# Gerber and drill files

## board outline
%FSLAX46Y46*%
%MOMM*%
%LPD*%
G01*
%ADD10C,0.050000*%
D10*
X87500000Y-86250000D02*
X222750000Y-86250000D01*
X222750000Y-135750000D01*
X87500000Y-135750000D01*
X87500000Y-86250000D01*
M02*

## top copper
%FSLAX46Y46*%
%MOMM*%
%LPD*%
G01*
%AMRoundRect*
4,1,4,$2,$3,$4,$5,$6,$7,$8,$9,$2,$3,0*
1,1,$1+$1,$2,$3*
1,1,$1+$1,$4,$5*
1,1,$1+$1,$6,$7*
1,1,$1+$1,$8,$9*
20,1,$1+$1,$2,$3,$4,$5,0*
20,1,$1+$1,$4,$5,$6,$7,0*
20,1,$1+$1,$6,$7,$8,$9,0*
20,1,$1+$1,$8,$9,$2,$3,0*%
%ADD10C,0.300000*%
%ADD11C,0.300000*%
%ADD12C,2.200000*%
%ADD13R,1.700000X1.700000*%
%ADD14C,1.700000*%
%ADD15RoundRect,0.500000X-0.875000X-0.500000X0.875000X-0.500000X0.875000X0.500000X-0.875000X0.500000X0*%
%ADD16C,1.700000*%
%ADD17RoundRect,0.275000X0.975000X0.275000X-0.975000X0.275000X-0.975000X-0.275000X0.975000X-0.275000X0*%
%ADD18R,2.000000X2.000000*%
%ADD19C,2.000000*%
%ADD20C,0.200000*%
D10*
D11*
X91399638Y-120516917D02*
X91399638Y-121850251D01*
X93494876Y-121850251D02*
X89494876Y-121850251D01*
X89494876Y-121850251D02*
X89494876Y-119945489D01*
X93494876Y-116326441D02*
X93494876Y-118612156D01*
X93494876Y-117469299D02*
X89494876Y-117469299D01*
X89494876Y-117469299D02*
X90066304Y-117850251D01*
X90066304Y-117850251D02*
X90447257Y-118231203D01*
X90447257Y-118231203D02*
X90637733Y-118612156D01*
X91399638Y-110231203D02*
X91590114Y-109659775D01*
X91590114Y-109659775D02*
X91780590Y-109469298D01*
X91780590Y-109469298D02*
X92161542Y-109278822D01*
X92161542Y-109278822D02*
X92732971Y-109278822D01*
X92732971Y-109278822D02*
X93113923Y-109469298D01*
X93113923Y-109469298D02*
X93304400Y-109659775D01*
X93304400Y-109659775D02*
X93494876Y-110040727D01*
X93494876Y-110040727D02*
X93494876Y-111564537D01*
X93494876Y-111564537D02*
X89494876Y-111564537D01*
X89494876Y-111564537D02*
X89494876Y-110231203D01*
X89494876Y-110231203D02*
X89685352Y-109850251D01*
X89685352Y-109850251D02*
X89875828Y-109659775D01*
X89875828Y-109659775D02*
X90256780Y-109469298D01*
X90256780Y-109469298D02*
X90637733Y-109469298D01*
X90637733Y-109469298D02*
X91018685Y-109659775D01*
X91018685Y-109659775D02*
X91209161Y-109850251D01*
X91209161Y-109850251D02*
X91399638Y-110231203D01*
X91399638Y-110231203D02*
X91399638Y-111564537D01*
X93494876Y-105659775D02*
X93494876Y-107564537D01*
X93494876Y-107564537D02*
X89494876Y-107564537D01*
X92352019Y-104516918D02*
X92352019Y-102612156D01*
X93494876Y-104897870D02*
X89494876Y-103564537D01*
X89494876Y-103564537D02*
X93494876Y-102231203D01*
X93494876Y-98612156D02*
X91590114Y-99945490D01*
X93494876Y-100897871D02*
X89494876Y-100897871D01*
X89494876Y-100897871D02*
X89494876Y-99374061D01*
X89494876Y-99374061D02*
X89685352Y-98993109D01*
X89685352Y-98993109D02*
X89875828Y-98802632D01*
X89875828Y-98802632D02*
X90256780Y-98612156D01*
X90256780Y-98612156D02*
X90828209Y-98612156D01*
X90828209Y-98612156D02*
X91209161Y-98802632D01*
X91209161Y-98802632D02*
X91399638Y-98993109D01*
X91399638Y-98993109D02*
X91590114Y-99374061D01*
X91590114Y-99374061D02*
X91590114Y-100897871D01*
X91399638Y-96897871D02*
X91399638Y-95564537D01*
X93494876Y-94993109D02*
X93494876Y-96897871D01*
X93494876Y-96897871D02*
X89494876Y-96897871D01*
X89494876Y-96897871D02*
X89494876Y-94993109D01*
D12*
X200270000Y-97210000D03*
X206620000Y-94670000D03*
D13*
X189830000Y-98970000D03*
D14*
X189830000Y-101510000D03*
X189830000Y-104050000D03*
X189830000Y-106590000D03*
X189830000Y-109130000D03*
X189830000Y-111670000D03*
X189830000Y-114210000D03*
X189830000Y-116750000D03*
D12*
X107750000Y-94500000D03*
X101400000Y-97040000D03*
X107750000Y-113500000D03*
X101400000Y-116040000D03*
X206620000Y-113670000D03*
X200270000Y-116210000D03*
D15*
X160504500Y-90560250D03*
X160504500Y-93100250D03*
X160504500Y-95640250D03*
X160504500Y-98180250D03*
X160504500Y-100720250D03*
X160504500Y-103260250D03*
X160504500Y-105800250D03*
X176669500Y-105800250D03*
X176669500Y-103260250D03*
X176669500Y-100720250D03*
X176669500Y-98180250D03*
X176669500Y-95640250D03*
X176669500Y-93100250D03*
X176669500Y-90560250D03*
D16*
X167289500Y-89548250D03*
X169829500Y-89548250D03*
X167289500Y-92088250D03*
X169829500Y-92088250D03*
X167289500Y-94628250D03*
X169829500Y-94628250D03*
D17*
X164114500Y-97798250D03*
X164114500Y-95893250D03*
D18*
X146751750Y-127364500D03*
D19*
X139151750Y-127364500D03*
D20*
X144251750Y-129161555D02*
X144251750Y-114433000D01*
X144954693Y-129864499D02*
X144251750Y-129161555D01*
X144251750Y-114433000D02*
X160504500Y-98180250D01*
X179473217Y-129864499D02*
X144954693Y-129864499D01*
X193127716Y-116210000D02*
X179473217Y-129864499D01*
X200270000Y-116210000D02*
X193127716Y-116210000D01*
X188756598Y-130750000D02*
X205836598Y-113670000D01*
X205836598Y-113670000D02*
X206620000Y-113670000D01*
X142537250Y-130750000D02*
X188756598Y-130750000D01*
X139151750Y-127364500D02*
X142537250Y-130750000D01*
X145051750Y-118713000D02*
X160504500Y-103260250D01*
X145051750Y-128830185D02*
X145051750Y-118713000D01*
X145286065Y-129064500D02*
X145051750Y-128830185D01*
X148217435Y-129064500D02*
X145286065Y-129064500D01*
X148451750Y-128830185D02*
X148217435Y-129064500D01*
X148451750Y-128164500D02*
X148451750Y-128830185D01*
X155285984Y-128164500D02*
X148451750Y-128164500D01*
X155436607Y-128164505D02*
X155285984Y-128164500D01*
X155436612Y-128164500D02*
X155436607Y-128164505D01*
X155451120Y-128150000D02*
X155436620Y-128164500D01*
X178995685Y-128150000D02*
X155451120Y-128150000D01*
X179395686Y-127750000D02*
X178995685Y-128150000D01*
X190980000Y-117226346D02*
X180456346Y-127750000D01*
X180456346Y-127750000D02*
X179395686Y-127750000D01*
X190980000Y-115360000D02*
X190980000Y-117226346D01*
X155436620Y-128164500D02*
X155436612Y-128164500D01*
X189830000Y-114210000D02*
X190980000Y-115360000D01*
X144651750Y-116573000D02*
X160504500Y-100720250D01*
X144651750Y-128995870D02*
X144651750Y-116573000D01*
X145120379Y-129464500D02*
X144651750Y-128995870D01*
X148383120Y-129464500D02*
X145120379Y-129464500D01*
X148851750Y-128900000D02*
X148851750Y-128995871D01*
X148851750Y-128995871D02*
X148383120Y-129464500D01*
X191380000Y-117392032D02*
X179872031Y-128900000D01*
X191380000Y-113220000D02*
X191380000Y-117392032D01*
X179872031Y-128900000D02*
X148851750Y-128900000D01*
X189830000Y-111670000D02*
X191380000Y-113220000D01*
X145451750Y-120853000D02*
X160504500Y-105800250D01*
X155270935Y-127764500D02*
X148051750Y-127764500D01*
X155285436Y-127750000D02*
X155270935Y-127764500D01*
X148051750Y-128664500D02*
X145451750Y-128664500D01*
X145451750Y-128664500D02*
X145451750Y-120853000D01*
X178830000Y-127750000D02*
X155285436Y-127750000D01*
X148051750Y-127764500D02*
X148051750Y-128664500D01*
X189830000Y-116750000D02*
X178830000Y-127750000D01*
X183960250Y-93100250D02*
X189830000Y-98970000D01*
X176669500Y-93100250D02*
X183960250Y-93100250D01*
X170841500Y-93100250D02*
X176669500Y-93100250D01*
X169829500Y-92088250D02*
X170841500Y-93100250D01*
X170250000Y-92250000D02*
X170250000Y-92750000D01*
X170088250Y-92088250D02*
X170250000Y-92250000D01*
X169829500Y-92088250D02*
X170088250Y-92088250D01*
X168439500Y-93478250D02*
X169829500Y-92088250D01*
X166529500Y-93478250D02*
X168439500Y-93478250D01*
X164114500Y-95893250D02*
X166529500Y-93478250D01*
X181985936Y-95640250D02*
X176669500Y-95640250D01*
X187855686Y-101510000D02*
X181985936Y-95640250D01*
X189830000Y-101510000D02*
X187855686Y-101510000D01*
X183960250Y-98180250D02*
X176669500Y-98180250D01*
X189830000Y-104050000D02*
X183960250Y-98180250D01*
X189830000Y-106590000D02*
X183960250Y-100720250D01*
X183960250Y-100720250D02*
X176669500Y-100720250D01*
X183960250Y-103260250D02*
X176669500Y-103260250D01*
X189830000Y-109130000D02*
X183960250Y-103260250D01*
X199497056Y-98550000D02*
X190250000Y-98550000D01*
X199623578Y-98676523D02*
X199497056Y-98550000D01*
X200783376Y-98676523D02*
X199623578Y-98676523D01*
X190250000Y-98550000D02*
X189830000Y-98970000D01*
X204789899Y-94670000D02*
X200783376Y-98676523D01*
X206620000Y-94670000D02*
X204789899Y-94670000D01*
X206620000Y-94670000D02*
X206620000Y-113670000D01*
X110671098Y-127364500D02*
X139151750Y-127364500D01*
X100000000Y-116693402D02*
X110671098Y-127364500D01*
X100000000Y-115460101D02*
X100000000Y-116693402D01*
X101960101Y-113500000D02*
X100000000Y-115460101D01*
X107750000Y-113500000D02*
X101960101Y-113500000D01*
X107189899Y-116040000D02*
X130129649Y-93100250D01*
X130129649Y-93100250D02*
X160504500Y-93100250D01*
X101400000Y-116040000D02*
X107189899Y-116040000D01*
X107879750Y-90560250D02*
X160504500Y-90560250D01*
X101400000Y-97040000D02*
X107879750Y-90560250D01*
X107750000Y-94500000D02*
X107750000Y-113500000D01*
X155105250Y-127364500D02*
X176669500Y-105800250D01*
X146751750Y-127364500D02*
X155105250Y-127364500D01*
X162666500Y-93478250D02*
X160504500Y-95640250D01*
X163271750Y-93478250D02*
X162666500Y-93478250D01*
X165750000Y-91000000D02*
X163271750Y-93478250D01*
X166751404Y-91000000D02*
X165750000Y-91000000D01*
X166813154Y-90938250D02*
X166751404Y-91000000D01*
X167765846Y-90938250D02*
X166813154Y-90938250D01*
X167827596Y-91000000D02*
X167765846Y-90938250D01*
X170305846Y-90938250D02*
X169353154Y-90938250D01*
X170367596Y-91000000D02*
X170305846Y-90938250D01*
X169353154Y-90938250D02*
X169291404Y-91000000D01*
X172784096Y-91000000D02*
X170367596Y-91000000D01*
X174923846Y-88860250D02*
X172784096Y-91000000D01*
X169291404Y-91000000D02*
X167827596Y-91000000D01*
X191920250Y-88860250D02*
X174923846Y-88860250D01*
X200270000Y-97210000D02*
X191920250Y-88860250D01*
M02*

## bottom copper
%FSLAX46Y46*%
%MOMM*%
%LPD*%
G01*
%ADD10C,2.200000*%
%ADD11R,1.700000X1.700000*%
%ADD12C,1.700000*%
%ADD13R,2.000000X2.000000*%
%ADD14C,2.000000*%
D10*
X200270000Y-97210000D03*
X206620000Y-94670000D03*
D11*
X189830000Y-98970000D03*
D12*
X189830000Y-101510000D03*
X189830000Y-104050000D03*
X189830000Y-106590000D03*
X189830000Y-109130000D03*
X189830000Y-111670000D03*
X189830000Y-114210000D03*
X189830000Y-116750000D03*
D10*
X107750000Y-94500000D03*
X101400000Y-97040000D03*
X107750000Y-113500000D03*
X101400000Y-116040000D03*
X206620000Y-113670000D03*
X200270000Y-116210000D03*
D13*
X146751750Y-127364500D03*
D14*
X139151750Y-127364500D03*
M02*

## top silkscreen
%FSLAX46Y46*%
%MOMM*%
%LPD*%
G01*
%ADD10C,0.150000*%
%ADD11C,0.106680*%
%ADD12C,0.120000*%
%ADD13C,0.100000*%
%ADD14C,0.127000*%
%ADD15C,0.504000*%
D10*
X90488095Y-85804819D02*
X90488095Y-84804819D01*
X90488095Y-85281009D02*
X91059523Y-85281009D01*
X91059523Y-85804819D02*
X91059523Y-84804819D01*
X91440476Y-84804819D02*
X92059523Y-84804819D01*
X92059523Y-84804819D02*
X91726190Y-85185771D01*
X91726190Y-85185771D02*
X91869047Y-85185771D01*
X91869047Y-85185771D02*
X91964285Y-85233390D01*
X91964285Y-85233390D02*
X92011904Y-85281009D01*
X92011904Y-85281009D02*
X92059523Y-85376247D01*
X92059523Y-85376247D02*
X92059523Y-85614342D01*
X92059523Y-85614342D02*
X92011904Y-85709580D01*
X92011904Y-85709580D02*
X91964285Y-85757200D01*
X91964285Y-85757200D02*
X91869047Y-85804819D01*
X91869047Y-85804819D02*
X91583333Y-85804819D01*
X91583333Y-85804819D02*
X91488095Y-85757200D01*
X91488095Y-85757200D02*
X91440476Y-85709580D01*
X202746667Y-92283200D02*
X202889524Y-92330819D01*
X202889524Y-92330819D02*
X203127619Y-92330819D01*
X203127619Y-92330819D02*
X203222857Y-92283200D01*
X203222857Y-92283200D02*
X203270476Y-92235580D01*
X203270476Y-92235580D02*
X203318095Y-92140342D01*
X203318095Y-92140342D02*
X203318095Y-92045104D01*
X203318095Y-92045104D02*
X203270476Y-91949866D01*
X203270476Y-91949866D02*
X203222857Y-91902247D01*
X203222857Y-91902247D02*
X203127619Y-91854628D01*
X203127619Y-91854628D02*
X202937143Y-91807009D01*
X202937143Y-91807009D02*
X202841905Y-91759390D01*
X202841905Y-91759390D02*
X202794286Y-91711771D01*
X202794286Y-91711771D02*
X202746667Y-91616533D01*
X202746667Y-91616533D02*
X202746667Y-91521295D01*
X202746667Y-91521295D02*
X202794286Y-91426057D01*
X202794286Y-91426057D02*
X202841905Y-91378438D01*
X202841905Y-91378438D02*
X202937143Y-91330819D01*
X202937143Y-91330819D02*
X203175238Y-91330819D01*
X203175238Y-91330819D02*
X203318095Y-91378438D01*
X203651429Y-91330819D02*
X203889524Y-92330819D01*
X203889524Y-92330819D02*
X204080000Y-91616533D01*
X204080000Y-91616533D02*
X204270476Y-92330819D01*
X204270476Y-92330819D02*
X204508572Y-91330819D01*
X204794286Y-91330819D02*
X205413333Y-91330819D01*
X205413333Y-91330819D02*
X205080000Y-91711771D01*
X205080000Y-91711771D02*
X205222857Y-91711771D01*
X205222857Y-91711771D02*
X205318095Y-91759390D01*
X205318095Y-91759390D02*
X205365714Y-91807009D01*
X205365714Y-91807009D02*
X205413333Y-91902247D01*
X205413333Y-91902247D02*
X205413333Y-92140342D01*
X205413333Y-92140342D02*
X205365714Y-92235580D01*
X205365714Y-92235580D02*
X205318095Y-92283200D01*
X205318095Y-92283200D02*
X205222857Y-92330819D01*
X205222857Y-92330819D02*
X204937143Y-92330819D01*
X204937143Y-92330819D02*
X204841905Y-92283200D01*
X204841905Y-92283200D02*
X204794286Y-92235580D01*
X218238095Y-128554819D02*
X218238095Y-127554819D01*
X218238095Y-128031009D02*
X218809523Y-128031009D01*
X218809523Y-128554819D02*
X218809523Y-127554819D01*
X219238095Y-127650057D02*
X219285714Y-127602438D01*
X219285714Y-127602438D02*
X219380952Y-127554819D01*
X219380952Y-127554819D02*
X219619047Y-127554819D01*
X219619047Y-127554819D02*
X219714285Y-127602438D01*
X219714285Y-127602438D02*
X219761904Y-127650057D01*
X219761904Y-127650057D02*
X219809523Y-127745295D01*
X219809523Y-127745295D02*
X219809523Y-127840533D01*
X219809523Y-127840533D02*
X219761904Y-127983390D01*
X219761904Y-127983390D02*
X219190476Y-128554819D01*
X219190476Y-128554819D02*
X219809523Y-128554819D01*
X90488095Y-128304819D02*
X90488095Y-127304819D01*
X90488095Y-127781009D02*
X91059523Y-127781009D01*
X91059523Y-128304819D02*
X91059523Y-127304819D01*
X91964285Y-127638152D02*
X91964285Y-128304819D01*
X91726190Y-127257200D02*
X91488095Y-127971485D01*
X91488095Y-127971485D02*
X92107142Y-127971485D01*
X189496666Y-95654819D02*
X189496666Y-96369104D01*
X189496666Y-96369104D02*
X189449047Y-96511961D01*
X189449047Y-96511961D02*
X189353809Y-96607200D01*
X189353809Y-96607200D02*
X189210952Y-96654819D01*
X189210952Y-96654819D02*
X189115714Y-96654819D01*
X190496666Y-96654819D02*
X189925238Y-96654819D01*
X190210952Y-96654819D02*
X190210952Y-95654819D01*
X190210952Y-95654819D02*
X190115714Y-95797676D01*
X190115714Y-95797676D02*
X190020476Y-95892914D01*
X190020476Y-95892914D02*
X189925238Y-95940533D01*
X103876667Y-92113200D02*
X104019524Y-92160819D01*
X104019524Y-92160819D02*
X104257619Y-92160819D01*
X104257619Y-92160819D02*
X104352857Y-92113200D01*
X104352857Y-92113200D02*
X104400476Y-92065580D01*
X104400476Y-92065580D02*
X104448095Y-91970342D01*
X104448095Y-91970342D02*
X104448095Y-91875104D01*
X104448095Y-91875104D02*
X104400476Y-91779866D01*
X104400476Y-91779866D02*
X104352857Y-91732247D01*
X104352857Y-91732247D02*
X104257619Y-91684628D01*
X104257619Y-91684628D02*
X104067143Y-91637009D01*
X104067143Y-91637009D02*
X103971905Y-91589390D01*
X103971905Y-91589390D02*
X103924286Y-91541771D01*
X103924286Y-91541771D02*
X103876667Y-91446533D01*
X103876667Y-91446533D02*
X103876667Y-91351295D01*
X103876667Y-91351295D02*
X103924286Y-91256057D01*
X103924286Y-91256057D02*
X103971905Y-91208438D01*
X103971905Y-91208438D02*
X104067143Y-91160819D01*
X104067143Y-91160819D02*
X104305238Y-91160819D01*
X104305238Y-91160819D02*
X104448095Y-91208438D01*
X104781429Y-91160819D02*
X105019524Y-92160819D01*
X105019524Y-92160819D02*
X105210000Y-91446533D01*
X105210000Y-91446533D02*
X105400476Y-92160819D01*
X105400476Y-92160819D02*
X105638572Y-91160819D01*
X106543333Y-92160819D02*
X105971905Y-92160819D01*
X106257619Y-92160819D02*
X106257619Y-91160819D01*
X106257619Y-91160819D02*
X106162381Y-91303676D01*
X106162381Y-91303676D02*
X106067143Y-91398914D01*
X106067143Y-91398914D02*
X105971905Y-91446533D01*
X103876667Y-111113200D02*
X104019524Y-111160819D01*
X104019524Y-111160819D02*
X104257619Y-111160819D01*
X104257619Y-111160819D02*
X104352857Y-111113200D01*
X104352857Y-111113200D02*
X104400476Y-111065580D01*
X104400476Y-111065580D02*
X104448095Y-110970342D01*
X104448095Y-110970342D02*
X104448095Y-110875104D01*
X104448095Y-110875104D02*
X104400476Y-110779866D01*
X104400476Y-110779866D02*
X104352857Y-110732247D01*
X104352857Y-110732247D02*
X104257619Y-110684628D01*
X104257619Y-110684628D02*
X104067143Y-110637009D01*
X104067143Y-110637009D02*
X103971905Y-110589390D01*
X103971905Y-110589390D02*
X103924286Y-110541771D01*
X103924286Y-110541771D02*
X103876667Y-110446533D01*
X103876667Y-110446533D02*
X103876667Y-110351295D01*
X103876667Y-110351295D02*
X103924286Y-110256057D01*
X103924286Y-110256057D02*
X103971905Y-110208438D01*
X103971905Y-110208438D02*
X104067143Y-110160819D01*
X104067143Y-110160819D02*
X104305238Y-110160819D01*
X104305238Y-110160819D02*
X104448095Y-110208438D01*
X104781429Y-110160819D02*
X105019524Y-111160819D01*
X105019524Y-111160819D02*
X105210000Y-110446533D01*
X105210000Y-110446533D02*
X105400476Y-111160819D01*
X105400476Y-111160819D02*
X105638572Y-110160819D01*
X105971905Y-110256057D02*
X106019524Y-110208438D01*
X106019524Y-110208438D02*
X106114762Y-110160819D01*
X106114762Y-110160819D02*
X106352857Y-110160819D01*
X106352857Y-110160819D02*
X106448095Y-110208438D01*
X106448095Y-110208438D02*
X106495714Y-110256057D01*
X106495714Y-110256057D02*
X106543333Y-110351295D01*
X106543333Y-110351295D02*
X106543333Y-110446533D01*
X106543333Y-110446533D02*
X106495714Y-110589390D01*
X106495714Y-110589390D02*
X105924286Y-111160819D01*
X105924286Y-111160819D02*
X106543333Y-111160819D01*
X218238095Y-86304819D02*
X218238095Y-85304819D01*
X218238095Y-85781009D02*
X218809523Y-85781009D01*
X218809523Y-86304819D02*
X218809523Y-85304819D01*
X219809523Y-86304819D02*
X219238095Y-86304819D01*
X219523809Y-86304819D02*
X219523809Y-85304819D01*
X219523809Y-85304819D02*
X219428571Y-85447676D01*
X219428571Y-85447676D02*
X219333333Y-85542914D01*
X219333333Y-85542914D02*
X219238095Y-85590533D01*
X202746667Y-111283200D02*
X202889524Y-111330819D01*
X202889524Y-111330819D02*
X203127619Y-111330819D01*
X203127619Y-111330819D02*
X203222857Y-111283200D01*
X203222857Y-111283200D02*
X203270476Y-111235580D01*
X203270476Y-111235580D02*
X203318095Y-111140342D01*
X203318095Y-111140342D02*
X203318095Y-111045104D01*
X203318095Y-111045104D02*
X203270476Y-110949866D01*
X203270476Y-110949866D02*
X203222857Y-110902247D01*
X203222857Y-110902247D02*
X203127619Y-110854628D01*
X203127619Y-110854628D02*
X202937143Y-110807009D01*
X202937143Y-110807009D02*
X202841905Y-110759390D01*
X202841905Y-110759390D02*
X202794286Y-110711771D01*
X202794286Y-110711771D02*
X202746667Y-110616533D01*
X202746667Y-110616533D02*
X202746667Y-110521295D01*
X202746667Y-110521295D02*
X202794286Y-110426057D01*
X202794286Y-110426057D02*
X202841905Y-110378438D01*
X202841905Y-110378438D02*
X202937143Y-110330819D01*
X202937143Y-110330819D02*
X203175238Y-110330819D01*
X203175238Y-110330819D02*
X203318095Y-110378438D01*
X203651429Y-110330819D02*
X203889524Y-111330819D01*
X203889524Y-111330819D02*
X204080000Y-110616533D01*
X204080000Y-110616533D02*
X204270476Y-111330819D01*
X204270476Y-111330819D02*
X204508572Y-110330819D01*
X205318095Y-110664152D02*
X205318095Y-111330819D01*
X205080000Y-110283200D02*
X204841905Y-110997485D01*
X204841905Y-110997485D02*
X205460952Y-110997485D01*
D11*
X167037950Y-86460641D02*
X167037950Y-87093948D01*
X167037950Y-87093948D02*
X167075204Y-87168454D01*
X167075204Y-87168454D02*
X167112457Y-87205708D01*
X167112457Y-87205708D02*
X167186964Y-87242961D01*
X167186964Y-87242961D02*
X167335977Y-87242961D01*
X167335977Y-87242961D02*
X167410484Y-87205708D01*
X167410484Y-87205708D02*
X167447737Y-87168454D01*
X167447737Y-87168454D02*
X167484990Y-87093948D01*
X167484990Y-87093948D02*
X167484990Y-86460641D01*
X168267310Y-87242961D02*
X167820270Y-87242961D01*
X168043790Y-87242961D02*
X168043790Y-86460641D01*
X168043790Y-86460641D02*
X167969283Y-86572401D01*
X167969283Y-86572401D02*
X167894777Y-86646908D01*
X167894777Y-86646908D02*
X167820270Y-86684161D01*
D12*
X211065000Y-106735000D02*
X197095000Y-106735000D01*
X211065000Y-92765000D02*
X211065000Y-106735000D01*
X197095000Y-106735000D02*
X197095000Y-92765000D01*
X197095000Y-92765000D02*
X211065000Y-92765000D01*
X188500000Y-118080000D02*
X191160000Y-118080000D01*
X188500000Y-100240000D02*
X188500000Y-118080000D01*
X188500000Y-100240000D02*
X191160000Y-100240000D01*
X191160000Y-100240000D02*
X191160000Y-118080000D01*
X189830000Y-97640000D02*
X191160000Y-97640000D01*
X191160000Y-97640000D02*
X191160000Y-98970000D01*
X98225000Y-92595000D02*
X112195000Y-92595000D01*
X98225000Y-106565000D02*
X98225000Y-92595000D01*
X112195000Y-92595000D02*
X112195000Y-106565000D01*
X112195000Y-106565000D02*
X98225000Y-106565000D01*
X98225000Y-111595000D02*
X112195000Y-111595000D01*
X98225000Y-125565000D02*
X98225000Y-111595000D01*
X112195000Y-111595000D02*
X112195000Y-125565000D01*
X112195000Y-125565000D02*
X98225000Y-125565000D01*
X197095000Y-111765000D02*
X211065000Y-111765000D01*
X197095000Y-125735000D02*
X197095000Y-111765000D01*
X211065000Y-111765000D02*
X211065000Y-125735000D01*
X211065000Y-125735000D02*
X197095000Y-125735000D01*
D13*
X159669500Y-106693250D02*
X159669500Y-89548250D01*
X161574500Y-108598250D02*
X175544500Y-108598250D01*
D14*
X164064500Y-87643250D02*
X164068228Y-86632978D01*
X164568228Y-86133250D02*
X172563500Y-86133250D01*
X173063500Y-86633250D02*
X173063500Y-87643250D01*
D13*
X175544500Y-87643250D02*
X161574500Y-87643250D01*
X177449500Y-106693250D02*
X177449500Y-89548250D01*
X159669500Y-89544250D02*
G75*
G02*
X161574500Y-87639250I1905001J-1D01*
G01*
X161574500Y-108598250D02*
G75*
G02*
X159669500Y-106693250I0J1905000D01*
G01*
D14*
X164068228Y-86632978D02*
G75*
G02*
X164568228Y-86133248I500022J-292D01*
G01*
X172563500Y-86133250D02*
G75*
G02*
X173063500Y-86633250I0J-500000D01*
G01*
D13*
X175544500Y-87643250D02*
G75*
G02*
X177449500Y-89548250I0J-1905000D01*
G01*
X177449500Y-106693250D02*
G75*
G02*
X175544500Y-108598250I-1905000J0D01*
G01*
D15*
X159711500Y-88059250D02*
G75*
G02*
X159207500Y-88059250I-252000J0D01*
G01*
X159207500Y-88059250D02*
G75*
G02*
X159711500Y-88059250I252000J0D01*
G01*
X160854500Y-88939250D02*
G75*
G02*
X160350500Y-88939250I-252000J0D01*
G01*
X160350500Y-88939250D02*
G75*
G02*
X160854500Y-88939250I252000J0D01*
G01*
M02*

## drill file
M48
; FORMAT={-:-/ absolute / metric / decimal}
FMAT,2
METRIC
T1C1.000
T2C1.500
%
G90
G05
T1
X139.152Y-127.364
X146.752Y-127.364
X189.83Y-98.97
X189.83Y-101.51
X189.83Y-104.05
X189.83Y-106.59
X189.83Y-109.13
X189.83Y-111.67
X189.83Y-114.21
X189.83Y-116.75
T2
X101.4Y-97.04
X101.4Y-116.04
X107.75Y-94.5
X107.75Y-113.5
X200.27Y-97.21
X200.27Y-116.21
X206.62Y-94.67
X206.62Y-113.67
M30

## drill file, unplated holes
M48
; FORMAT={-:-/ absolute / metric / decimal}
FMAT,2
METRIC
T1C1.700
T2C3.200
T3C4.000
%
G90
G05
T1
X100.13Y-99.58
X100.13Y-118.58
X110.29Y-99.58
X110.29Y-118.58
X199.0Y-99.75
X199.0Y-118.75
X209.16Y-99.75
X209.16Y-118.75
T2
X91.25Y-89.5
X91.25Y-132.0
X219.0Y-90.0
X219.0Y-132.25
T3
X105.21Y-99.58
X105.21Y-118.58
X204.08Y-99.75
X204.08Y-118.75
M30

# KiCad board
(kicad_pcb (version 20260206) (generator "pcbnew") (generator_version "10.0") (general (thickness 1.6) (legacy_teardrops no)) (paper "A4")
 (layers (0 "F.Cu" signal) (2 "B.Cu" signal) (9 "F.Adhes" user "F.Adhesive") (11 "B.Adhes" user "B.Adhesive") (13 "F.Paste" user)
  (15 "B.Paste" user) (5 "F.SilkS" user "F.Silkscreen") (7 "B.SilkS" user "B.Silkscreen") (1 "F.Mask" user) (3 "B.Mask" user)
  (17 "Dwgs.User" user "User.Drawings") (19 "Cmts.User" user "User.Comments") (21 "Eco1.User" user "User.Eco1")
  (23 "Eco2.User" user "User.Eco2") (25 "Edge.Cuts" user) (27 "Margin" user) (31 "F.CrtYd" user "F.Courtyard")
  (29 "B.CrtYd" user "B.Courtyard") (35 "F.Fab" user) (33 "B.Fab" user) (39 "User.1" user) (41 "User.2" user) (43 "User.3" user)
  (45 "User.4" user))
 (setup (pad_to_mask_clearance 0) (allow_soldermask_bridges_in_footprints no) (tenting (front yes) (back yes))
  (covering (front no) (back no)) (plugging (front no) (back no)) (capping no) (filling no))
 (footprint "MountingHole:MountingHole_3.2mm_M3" (layer "F.Cu") (at 219 132.25)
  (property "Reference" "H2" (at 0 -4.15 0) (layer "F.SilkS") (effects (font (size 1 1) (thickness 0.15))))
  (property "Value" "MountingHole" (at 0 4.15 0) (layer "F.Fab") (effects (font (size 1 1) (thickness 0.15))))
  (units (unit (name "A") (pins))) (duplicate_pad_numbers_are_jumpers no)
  (pad "" np_thru_hole circle (at 0 0) (size 3.2 3.2) (drill 3.2) (layers "*.Cu" "*.Mask")))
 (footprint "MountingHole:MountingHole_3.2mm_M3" (layer "F.Cu") (at 91.25 132)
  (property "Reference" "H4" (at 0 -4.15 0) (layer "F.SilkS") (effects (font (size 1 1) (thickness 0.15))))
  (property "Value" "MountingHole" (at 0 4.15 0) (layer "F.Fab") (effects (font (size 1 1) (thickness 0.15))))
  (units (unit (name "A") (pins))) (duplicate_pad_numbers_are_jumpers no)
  (pad "" np_thru_hole circle (at 0 0) (size 3.2 3.2) (drill 3.2) (layers "*.Cu" "*.Mask")))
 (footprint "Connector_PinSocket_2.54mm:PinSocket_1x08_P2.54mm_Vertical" (layer "F.Cu") (at 189.83 98.97)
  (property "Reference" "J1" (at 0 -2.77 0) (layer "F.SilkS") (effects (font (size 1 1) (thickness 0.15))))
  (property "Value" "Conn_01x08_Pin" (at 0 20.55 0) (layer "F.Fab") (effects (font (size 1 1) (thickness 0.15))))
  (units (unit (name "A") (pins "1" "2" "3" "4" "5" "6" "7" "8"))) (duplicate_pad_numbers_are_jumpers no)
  (fp_line (start -1.33 1.27) (end -1.33 19.11) (stroke (width 0.12) (type solid)) (layer "F.SilkS"))
  (fp_line (start -1.33 1.27) (end 1.33 1.27) (stroke (width 0.12) (type solid)) (layer "F.SilkS"))
  (fp_line (start -1.33 19.11) (end 1.33 19.11) (stroke (width 0.12) (type solid)) (layer "F.SilkS"))
  (fp_line (start 0 -1.33) (end 1.33 -1.33) (stroke (width 0.12) (type solid)) (layer "F.SilkS"))
  (fp_line (start 1.33 -1.33) (end 1.33 0) (stroke (width 0.12) (type solid)) (layer "F.SilkS"))
  (fp_line (start 1.33 1.27) (end 1.33 19.11) (stroke (width 0.12) (type solid)) (layer "F.SilkS"))
  (pad "1" thru_hole rect (at 0 0) (size 1.7 1.7) (drill 1) (layers "*.Cu" "*.Mask") (remove_unused_layers no) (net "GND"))
  (pad "2" thru_hole circle (at 0 2.54) (size 1.7 1.7) (drill 1) (layers "*.Cu" "*.Mask") (remove_unused_layers no) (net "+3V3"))
  (pad "3" thru_hole circle (at 0 5.08) (size 1.7 1.7) (drill 1) (layers "*.Cu" "*.Mask") (remove_unused_layers no) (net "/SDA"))
  (pad "4" thru_hole circle (at 0 7.62) (size 1.7 1.7) (drill 1) (layers "*.Cu" "*.Mask") (remove_unused_layers no) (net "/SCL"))
  (pad "5" thru_hole circle (at 0 10.16) (size 1.7 1.7) (drill 1) (layers "*.Cu" "*.Mask") (remove_unused_layers no) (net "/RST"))
  (pad "6" thru_hole circle (at 0 12.7) (size 1.7 1.7) (drill 1) (layers "*.Cu" "*.Mask") (remove_unused_layers no) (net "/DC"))
  (pad "7" thru_hole circle (at 0 15.24) (size 1.7 1.7) (drill 1) (layers "*.Cu" "*.Mask") (remove_unused_layers no) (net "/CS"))
  (pad "8" thru_hole circle (at 0 17.78) (size 1.7 1.7) (drill 1) (layers "*.Cu" "*.Mask") (remove_unused_layers no) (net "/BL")))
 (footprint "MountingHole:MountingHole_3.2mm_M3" (layer "F.Cu") (at 91.25 89.5)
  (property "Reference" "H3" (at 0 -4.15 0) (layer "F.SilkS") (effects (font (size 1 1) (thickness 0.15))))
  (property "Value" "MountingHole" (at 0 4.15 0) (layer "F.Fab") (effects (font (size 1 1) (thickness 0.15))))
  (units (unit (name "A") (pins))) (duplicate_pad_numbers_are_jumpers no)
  (pad "" np_thru_hole circle (at 0 0) (size 3.2 3.2) (drill 3.2) (layers "*.Cu" "*.Mask")))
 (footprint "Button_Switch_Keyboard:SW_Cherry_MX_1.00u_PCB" (layer "F.Cu") (at 206.62 94.67)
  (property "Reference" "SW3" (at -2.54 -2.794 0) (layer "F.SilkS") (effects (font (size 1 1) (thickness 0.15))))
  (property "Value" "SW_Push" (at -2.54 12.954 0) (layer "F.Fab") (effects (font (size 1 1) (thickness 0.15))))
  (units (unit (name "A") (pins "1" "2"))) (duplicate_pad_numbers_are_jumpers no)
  (fp_line (start -9.525 -1.905) (end 4.445 -1.905) (stroke (width 0.12) (type solid)) (layer "F.SilkS"))
  (fp_line (start -9.525 12.065) (end -9.525 -1.905) (stroke (width 0.12) (type solid)) (layer "F.SilkS"))
  (fp_line (start 4.445 -1.905) (end 4.445 12.065) (stroke (width 0.12) (type solid)) (layer "F.SilkS"))
  (fp_line (start 4.445 12.065) (end -9.525 12.065) (stroke (width 0.12) (type solid)) (layer "F.SilkS"))
  (pad "" np_thru_hole circle (at -7.62 5.08) (size 1.7 1.7) (drill 1.7) (layers "*.Cu" "*.Mask"))
  (pad "" np_thru_hole circle (at -2.54 5.08) (size 4 4) (drill 4) (layers "*.Cu" "*.Mask"))
  (pad "" np_thru_hole circle (at 2.54 5.08) (size 1.7 1.7) (drill 1.7) (layers "*.Cu" "*.Mask"))
  (pad "1" thru_hole circle (at 0 0) (size 2.2 2.2) (drill 1.5) (layers "*.Cu" "*.Mask") (remove_unused_layers no) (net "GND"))
  (pad "2" thru_hole circle (at -6.35 2.54) (size 2.2 2.2) (drill 1.5) (layers "*.Cu" "*.Mask") (remove_unused_layers no)
   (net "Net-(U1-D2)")))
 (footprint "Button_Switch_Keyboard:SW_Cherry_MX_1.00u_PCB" (layer "F.Cu") (at 107.75 94.5)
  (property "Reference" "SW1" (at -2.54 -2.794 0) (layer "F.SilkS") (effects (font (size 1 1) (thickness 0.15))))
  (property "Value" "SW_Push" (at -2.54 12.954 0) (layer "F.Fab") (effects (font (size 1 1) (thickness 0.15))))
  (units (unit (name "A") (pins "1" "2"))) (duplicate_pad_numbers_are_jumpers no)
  (fp_line (start -9.525 -1.905) (end 4.445 -1.905) (stroke (width 0.12) (type solid)) (layer "F.SilkS"))
  (fp_line (start -9.525 12.065) (end -9.525 -1.905) (stroke (width 0.12) (type solid)) (layer "F.SilkS"))
  (fp_line (start 4.445 -1.905) (end 4.445 12.065) (stroke (width 0.12) (type solid)) (layer "F.SilkS"))
  (fp_line (start 4.445 12.065) (end -9.525 12.065) (stroke (width 0.12) (type solid)) (layer "F.SilkS"))
  (pad "" np_thru_hole circle (at -7.62 5.08) (size 1.7 1.7) (drill 1.7) (layers "*.Cu" "*.Mask"))
  (pad "" np_thru_hole circle (at -2.54 5.08) (size 4 4) (drill 4) (layers "*.Cu" "*.Mask"))
  (pad "" np_thru_hole circle (at 2.54 5.08) (size 1.7 1.7) (drill 1.7) (layers "*.Cu" "*.Mask"))
  (pad "1" thru_hole circle (at 0 0) (size 2.2 2.2) (drill 1.5) (layers "*.Cu" "*.Mask") (remove_unused_layers no) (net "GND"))
  (pad "2" thru_hole circle (at -6.35 2.54) (size 2.2 2.2) (drill 1.5) (layers "*.Cu" "*.Mask") (remove_unused_layers no)
   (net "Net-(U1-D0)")))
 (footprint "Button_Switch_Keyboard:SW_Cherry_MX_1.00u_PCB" (layer "F.Cu") (at 107.75 113.5)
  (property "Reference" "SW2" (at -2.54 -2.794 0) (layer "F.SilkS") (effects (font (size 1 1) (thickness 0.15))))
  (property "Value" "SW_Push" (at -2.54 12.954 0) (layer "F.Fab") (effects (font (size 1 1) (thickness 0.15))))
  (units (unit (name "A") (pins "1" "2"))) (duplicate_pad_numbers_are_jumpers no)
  (fp_line (start -9.525 -1.905) (end 4.445 -1.905) (stroke (width 0.12) (type solid)) (layer "F.SilkS"))
  (fp_line (start -9.525 12.065) (end -9.525 -1.905) (stroke (width 0.12) (type solid)) (layer "F.SilkS"))
  (fp_line (start 4.445 -1.905) (end 4.445 12.065) (stroke (width 0.12) (type solid)) (layer "F.SilkS"))
  (fp_line (start 4.445 12.065) (end -9.525 12.065) (stroke (width 0.12) (type solid)) (layer "F.SilkS"))
  (pad "" np_thru_hole circle (at -7.62 5.08) (size 1.7 1.7) (drill 1.7) (layers "*.Cu" "*.Mask"))
  (pad "" np_thru_hole circle (at -2.54 5.08) (size 4 4) (drill 4) (layers "*.Cu" "*.Mask"))
  (pad "" np_thru_hole circle (at 2.54 5.08) (size 1.7 1.7) (drill 1.7) (layers "*.Cu" "*.Mask"))
  (pad "1" thru_hole circle (at 0 0) (size 2.2 2.2) (drill 1.5) (layers "*.Cu" "*.Mask") (remove_unused_layers no) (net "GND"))
  (pad "2" thru_hole circle (at -6.35 2.54) (size 2.2 2.2) (drill 1.5) (layers "*.Cu" "*.Mask") (remove_unused_layers no)
   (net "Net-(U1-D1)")))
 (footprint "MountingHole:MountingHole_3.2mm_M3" (layer "F.Cu") (at 219 90)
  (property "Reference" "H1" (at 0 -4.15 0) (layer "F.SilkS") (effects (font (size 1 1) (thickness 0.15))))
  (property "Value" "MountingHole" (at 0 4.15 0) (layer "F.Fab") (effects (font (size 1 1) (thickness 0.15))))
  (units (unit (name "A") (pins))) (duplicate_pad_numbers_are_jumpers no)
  (pad "" np_thru_hole circle (at 0 0) (size 3.2 3.2) (drill 3.2) (layers "*.Cu" "*.Mask")))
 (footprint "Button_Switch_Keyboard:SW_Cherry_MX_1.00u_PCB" (layer "F.Cu") (at 206.62 113.67)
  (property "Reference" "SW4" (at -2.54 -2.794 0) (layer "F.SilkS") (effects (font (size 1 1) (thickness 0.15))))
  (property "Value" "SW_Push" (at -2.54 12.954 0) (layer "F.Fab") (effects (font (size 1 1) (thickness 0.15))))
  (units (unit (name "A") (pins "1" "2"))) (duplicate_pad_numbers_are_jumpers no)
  (fp_line (start -9.525 -1.905) (end 4.445 -1.905) (stroke (width 0.12) (type solid)) (layer "F.SilkS"))
  (fp_line (start -9.525 12.065) (end -9.525 -1.905) (stroke (width 0.12) (type solid)) (layer "F.SilkS"))
  (fp_line (start 4.445 -1.905) (end 4.445 12.065) (stroke (width 0.12) (type solid)) (layer "F.SilkS"))
  (fp_line (start 4.445 12.065) (end -9.525 12.065) (stroke (width 0.12) (type solid)) (layer "F.SilkS"))
  (pad "" np_thru_hole circle (at -7.62 5.08) (size 1.7 1.7) (drill 1.7) (layers "*.Cu" "*.Mask"))
  (pad "" np_thru_hole circle (at -2.54 5.08) (size 4 4) (drill 4) (layers "*.Cu" "*.Mask"))
  (pad "" np_thru_hole circle (at 2.54 5.08) (size 1.7 1.7) (drill 1.7) (layers "*.Cu" "*.Mask"))
  (pad "1" thru_hole circle (at 0 0) (size 2.2 2.2) (drill 1.5) (layers "*.Cu" "*.Mask") (remove_unused_layers no) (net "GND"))
  (pad "2" thru_hole circle (at -6.35 2.54) (size 2.2 2.2) (drill 1.5) (layers "*.Cu" "*.Mask") (remove_unused_layers no)
   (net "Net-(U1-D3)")))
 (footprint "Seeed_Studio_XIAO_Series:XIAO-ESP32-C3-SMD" (layer "F.Cu") (at 159.6695 108.68025)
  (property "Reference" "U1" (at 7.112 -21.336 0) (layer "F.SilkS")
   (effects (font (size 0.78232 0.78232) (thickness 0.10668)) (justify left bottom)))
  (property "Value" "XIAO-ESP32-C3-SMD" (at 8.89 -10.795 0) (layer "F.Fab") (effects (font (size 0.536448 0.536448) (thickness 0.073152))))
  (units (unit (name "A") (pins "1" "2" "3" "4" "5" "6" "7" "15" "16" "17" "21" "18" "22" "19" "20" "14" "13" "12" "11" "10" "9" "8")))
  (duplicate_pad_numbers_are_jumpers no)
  (fp_line (start 0 -1.987) (end 0 -19.132) (stroke (width 0.1) (type solid)) (layer "F.SilkS"))
  (fp_line (start 1.905 -0.082) (end 15.875 -0.082) (stroke (width 0.1) (type solid)) (layer "F.SilkS"))
  (fp_line (start 4.395 -21.037) (end 4.398728 -22.047272) (stroke (width 0.127) (type solid)) (layer "F.SilkS"))
  (fp_line (start 4.898728 -22.547) (end 12.894 -22.547) (stroke (width 0.127) (type solid)) (layer "F.SilkS"))
  (fp_line (start 13.394 -22.047) (end 13.394 -21.037) (stroke (width 0.127) (type solid)) (layer "F.SilkS"))
  (fp_line (start 15.875 -21.037) (end 1.905 -21.037) (stroke (width 0.1) (type solid)) (layer "F.SilkS"))
  (fp_line (start 17.78 -1.987) (end 17.78 -19.132) (stroke (width 0.1) (type solid)) (layer "F.SilkS"))
  (fp_arc (start 0 -19.136) (mid 0.557962 -20.483038) (end 1.905 -21.041) (stroke (width 0.1) (type solid)) (layer "F.SilkS"))
  (fp_arc (start 1.905 -0.082) (mid 0.557962 -0.639962) (end 0 -1.987) (stroke (width 0.1) (type solid)) (layer "F.SilkS"))
  (fp_arc (start 4.398728 -22.047272) (mid 4.545272 -22.40064) (end 4.898728 -22.547) (stroke (width 0.127) (type default))
   (layer "F.SilkS"))
  (fp_arc (start 12.894 -22.547) (mid 13.247553 -22.400553) (end 13.394 -22.047) (stroke (width 0.127) (type default)) (layer "F.SilkS"))
  (fp_arc (start 15.875 -21.037) (mid 17.222038 -20.479038) (end 17.78 -19.132) (stroke (width 0.1) (type solid)) (layer "F.SilkS"))
  (fp_arc (start 17.78 -1.987) (mid 17.222038 -0.639962) (end 15.875 -0.082) (stroke (width 0.1) (type solid)) (layer "F.SilkS"))
  (fp_circle (center -0.21 -20.621) (end -0.21 -20.875) (stroke (width 0.5) (type solid)) (fill yes) (layer "F.SilkS"))
  (fp_circle (center 0.933 -19.741) (end 0.933 -19.995) (stroke (width 0.5) (type solid)) (fill yes) (layer "F.SilkS"))
  (pad "1" smd roundrect (at 0.835 -18.12) (size 2.75 2) (layers "F.Cu" "F.Mask" "F.Paste") (roundrect_rratio 0.25) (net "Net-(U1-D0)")
   (solder_mask_margin 0.0508) (thermal_bridge_angle 45))
  (pad "2" smd roundrect (at 0.835 -15.58) (size 2.75 2) (layers "F.Cu" "F.Mask" "F.Paste") (roundrect_rratio 0.25) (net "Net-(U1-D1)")
   (solder_mask_margin 0.0508) (thermal_bridge_angle 45))
  (pad "3" smd roundrect (at 0.835 -13.04) (size 2.75 2) (layers "F.Cu" "F.Mask" "F.Paste") (roundrect_rratio 0.25) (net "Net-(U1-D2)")
   (solder_mask_margin 0.0508) (thermal_bridge_angle 45))
  (pad "4" smd roundrect (at 0.835 -10.5) (size 2.75 2) (layers "F.Cu" "F.Mask" "F.Paste") (roundrect_rratio 0.25) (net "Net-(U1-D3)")
   (solder_mask_margin 0.0508) (thermal_bridge_angle 45))
  (pad "5" smd roundrect (at 0.835 -7.96) (size 2.75 2) (layers "F.Cu" "F.Mask" "F.Paste") (roundrect_rratio 0.25) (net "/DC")
   (solder_mask_margin 0.0508) (thermal_bridge_angle 45))
  (pad "6" smd roundrect (at 0.835 -5.42) (size 2.75 2) (layers "F.Cu" "F.Mask" "F.Paste") (roundrect_rratio 0.25) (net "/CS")
   (solder_mask_margin 0.0508) (thermal_bridge_angle 45))
  (pad "7" smd roundrect (at 0.835 -2.88) (size 2.75 2) (layers "F.Cu" "F.Mask" "F.Paste") (roundrect_rratio 0.25) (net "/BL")
   (solder_mask_margin 0.0508) (thermal_bridge_angle 45))
  (pad "8" smd roundrect (at 17 -2.88) (size 2.75 2) (layers "F.Cu" "F.Mask" "F.Paste") (roundrect_rratio 0.25) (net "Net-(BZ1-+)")
   (solder_mask_margin 0.0508) (thermal_bridge_angle 45))
  (pad "9" smd roundrect (at 17 -5.42) (size 2.75 2) (layers "F.Cu" "F.Mask" "F.Paste") (roundrect_rratio 0.25) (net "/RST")
   (solder_mask_margin 0.0508) (thermal_bridge_angle 45))
  (pad "10" smd roundrect (at 17 -7.96) (size 2.75 2) (layers "F.Cu" "F.Mask" "F.Paste") (roundrect_rratio 0.25) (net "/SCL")
   (solder_mask_margin 0.0508) (thermal_bridge_angle 45))
  (pad "11" smd roundrect (at 17 -10.5) (size 2.75 2) (layers "F.Cu" "F.Mask" "F.Paste") (roundrect_rratio 0.25) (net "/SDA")
   (solder_mask_margin 0.0508) (thermal_bridge_angle 45))
  (pad "12" smd roundrect (at 17 -13.04) (size 2.75 2) (layers "F.Cu" "F.Mask" "F.Paste") (roundrect_rratio 0.25) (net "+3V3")
   (solder_mask_margin 0.0508) (thermal_bridge_angle 45))
  (pad "13" smd roundrect (at 17 -15.58) (size 2.75 2) (layers "F.Cu" "F.Mask" "F.Paste") (roundrect_rratio 0.25) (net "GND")
   (solder_mask_margin 0.0508) (thermal_bridge_angle 45))
  (pad "14" smd roundrect (at 17 -18.12) (size 2.75 2) (layers "F.Cu" "F.Mask" "F.Paste") (roundrect_rratio 0.25)
   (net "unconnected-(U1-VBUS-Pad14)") (solder_mask_margin 0.0508) (thermal_bridge_angle 45))
  (pad "15" smd circle (at 7.62 -19.132) (size 1.7 1.7) (layers "F.Cu" "F.Mask" "F.Paste") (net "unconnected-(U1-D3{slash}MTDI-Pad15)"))
  (pad "16" smd circle (at 10.16 -19.132) (size 1.7 1.7) (layers "F.Cu" "F.Mask" "F.Paste") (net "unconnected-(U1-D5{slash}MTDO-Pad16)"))
  (pad "17" smd circle (at 7.62 -16.592) (size 1.7 1.7) (layers "F.Cu" "F.Mask" "F.Paste") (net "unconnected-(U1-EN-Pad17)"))
  (pad "18" smd circle (at 10.16 -16.592) (size 1.7 1.7) (layers "F.Cu" "F.Mask" "F.Paste") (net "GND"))
  (pad "19" smd circle (at 7.62 -14.052) (size 1.7 1.7) (layers "F.Cu" "F.Mask" "F.Paste") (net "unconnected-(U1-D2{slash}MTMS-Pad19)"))
  (pad "20" smd circle (at 10.16 -14.052) (size 1.7 1.7) (layers "F.Cu" "F.Mask" "F.Paste") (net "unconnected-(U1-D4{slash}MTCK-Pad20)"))
  (pad "21" smd roundrect (at 4.445 -10.882 180) (size 2.5 1.1) (layers "F.Cu" "F.Mask" "F.Paste") (roundrect_rratio 0.25)
   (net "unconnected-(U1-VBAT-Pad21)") (thermal_bridge_angle 45))
  (pad "22" smd roundrect (at 4.445 -12.787 180) (size 2.5 1.1) (layers "F.Cu" "F.Mask" "F.Paste") (roundrect_rratio 0.25) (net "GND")
   (thermal_bridge_angle 45)))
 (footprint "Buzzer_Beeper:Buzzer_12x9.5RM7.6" (layer "B.Cu") (at 146.75175 127.3645 180)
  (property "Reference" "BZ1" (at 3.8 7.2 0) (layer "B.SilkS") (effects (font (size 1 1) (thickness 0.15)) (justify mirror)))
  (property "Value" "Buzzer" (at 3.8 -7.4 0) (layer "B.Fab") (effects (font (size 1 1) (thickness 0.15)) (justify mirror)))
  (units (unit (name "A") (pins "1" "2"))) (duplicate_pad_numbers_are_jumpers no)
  (pad "1" thru_hole rect (at 0 0 180) (size 2 2) (drill 1) (layers "*.Cu" "*.Mask") (remove_unused_layers no) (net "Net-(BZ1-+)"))
  (pad "2" thru_hole circle (at 7.6 0 180) (size 2 2) (drill 1) (layers "*.Cu" "*.Mask") (remove_unused_layers no) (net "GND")))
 (gr_rect (start 87.5 86.25) (end 222.75 135.75) (stroke (width 0.05) (type default)) (fill no) (layer "Edge.Cuts"))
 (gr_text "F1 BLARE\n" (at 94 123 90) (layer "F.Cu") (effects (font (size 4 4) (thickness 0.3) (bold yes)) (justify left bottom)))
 (segment (start 168.4395 93.47825) (end 169.8295 92.08825) (width 0.2) (layer "F.Cu") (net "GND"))
 (segment (start 206.62 94.67) (end 206.62 113.67) (width 0.2) (layer "F.Cu") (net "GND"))
 (segment (start 205.836598 113.67) (end 206.62 113.67) (width 0.2) (layer "F.Cu") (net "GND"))
 (segment (start 199.497056 98.55) (end 190.25 98.55) (width 0.2) (layer "F.Cu") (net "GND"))
 (segment (start 142.53725 130.75) (end 188.756598 130.75) (width 0.2) (layer "F.Cu") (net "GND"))
 (segment (start 100 116.693402) (end 110.671098 127.3645) (width 0.2) (layer "F.Cu") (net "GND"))
 (segment (start 100 115.460101) (end 100 116.693402) (width 0.2) (layer "F.Cu") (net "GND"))
 (segment (start 206.62 94.67) (end 204.789899 94.67) (width 0.2) (layer "F.Cu") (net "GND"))
 (segment (start 101.960101 113.5) (end 100 115.460101) (width 0.2) (layer "F.Cu") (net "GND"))
 (segment (start 169.8295 92.08825) (end 170.8415 93.10025) (width 0.2) (layer "F.Cu") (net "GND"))
 (segment (start 110.671098 127.3645) (end 139.15175 127.3645) (width 0.2) (layer "F.Cu") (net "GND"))
 (segment (start 199.623578 98.676523) (end 199.497056 98.55) (width 0.2) (layer "F.Cu") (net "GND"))
 (segment (start 200.783376 98.676523) (end 199.623578 98.676523) (width 0.2) (layer "F.Cu") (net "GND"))
 (segment (start 204.789899 94.67) (end 200.783376 98.676523) (width 0.2) (layer "F.Cu") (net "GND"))
 (segment (start 169.8295 92.08825) (end 170.08825 92.08825) (width 0.2) (layer "F.Cu") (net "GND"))
 (segment (start 107.75 94.5) (end 107.75 113.5) (width 0.2) (layer "F.Cu") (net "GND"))
 (segment (start 190.25 98.55) (end 189.83 98.97) (width 0.2) (layer "F.Cu") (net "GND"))
 (segment (start 166.5295 93.47825) (end 168.4395 93.47825) (width 0.2) (layer "F.Cu") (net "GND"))
 (segment (start 183.96025 93.10025) (end 189.83 98.97) (width 0.2) (layer "F.Cu") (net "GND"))
 (segment (start 170.08825 92.08825) (end 170.25 92.25) (width 0.2) (layer "F.Cu") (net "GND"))
 (segment (start 139.15175 127.3645) (end 142.53725 130.75) (width 0.2) (layer "F.Cu") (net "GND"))
 (segment (start 188.756598 130.75) (end 205.836598 113.67) (width 0.2) (layer "F.Cu") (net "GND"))
 (segment (start 170.25 92.25) (end 170.25 92.75) (width 0.2) (layer "F.Cu") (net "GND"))
 (segment (start 176.6695 93.10025) (end 183.96025 93.10025) (width 0.2) (layer "F.Cu") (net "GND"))
 (segment (start 107.75 113.5) (end 101.960101 113.5) (width 0.2) (layer "F.Cu") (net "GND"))
 (segment (start 164.1145 95.89325) (end 166.5295 93.47825) (width 0.2) (layer "F.Cu") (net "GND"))
 (segment (start 170.8415 93.10025) (end 176.6695 93.10025) (width 0.2) (layer "F.Cu") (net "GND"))
 (segment (start 181.985936 95.64025) (end 176.6695 95.64025) (width 0.2) (layer "F.Cu") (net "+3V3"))
 (segment (start 189.83 101.51) (end 187.855686 101.51) (width 0.2) (layer "F.Cu") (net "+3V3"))
 (segment (start 187.855686 101.51) (end 181.985936 95.64025) (width 0.2) (layer "F.Cu") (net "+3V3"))
 (segment (start 183.96025 98.18025) (end 176.6695 98.18025) (width 0.2) (layer "F.Cu") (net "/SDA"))
 (segment (start 189.83 104.05) (end 183.96025 98.18025) (width 0.2) (layer "F.Cu") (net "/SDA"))
 (segment (start 189.83 106.59) (end 183.96025 100.72025) (width 0.2) (layer "F.Cu") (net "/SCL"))
 (segment (start 183.96025 100.72025) (end 176.6695 100.72025) (width 0.2) (layer "F.Cu") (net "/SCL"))
 (segment (start 183.96025 103.26025) (end 176.6695 103.26025) (width 0.2) (layer "F.Cu") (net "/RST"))
 (segment (start 189.83 109.13) (end 183.96025 103.26025) (width 0.2) (layer "F.Cu") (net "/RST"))
 (segment (start 148.38312 129.4645) (end 145.120379 129.4645) (width 0.2) (layer "F.Cu") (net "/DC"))
 (segment (start 179.872031 128.9) (end 148.85175 128.9) (width 0.2) (layer "F.Cu") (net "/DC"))
 (segment (start 189.83 111.67) (end 191.38 113.22) (width 0.2) (layer "F.Cu") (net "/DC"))
 (segment (start 191.38 113.22) (end 191.38 117.392032) (width 0.2) (layer "F.Cu") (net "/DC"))
 (segment (start 144.65175 116.573) (end 160.5045 100.72025) (width 0.2) (layer "F.Cu") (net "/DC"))
 (segment (start 191.38 117.392032) (end 179.872031 128.9) (width 0.2) (layer "F.Cu") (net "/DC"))
 (segment (start 148.85175 128.995871) (end 148.38312 129.4645) (width 0.2) (layer "F.Cu") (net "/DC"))
 (segment (start 144.65175 128.99587) (end 144.65175 116.573) (width 0.2) (layer "F.Cu") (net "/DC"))
 (segment (start 148.85175 128.9) (end 148.85175 128.995871) (width 0.2) (layer "F.Cu") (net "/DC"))
 (segment (start 145.120379 129.4645) (end 144.65175 128.99587) (width 0.2) (layer "F.Cu") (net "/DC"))
 (segment (start 145.286065 129.0645) (end 145.05175 128.830185) (width 0.2) (layer "F.Cu") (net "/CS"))
 (segment (start 155.285984 128.1645) (end 148.45175 128.1645) (width 0.2) (layer "F.Cu") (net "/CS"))
 (segment (start 190.98 115.36) (end 190.98 117.226346) (width 0.2) (layer "F.Cu") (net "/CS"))
 (segment (start 179.395686 127.75) (end 178.995685 128.15) (width 0.2) (layer "F.Cu") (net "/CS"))
 (segment (start 148.217435 129.0645) (end 145.286065 129.0645) (width 0.2) (layer "F.Cu") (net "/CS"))
 (segment (start 148.45175 128.1645) (end 148.45175 128.830185) (width 0.2) (layer "F.Cu") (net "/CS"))
 (segment (start 178.995685 128.15) (end 155.45112 128.15) (width 0.2) (layer "F.Cu") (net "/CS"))
 (segment (start 189.83 114.21) (end 190.98 115.36) (width 0.2) (layer "F.Cu") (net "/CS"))
 (segment (start 180.456346 127.75) (end 179.395686 127.75) (width 0.2) (layer "F.Cu") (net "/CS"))
 (segment (start 148.45175 128.830185) (end 148.217435 129.0645) (width 0.2) (layer "F.Cu") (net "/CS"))
 (segment (start 190.98 117.226346) (end 180.456346 127.75) (width 0.2) (layer "F.Cu") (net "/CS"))
 (segment (start 155.45112 128.15) (end 155.43662 128.1645) (width 0.2) (layer "F.Cu") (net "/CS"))
 (segment (start 145.05175 118.713) (end 160.5045 103.26025) (width 0.2) (layer "F.Cu") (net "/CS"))
 (segment (start 155.436612 128.1645) (end 155.436607 128.164505) (width 0.2) (layer "F.Cu") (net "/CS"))
 (segment (start 155.43662 128.1645) (end 155.436612 128.1645) (width 0.2) (layer "F.Cu") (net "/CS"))
 (segment (start 155.436607 128.164505) (end 155.285984 128.1645) (width 0.2) (layer "F.Cu") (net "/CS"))
 (segment (start 145.05175 128.830185) (end 145.05175 118.713) (width 0.2) (layer "F.Cu") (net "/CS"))
 (segment (start 155.270935 127.7645) (end 148.05175 127.7645) (width 0.2) (layer "F.Cu") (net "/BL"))
 (segment (start 148.05175 127.7645) (end 148.05175 128.6645) (width 0.2) (layer "F.Cu") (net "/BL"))
 (segment (start 145.45175 120.853) (end 160.5045 105.80025) (width 0.2) (layer "F.Cu") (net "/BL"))
 (segment (start 178.83 127.75) (end 155.285436 127.75) (width 0.2) (layer "F.Cu") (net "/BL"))
 (segment (start 155.285436 127.75) (end 155.270935 127.7645) (width 0.2) (layer "F.Cu") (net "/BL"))
 (segment (start 145.45175 128.6645) (end 145.45175 120.853) (width 0.2) (layer "F.Cu") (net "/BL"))
 (segment (start 148.05175 128.6645) (end 145.45175 128.6645) (width 0.2) (layer "F.Cu") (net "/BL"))
 (segment (start 189.83 116.75) (end 178.83 127.75) (width 0.2) (layer "F.Cu") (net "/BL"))
 (segment (start 167.827596 91) (end 167.765846 90.93825) (width 0.2) (layer "F.Cu") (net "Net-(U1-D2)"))
 (segment (start 166.751404 91) (end 165.75 91) (width 0.2) (layer "F.Cu") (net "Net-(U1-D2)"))
 (segment (start 170.305846 90.93825) (end 169.353154 90.93825) (width 0.2) (layer "F.Cu") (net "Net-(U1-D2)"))
 (segment (start 191.92025 88.86025) (end 174.923846 88.86025) (width 0.2) (layer "F.Cu") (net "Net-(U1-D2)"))
 (segment (start 174.923846 88.86025) (end 172.784096 91) (width 0.2) (layer "F.Cu") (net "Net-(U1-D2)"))
 (segment (start 165.75 91) (end 163.27175 93.47825) (width 0.2) (layer "F.Cu") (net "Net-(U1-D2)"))
 (segment (start 172.784096 91) (end 170.367596 91) (width 0.2) (layer "F.Cu") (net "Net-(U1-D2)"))
 (segment (start 169.353154 90.93825) (end 169.291404 91) (width 0.2) (layer "F.Cu") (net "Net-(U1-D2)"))
 (segment (start 200.27 97.21) (end 191.92025 88.86025) (width 0.2) (layer "F.Cu") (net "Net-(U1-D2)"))
 (segment (start 169.291404 91) (end 167.827596 91) (width 0.2) (layer "F.Cu") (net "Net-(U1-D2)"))
 (segment (start 163.27175 93.47825) (end 162.6665 93.47825) (width 0.2) (layer "F.Cu") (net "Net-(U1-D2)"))
 (segment (start 167.765846 90.93825) (end 166.813154 90.93825) (width 0.2) (layer "F.Cu") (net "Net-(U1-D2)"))
 (segment (start 162.6665 93.47825) (end 160.5045 95.64025) (width 0.2) (layer "F.Cu") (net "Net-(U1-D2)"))
 (segment (start 166.813154 90.93825) (end 166.751404 91) (width 0.2) (layer "F.Cu") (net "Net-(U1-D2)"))
 (segment (start 170.367596 91) (end 170.305846 90.93825) (width 0.2) (layer "F.Cu") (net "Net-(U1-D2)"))
 (segment (start 101.4 97.04) (end 107.87975 90.56025) (width 0.2) (layer "F.Cu") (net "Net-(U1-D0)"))
 (segment (start 107.87975 90.56025) (end 160.5045 90.56025) (width 0.2) (layer "F.Cu") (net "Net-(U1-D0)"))
 (segment (start 130.129649 93.10025) (end 160.5045 93.10025) (width 0.2) (layer "F.Cu") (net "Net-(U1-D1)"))
 (segment (start 107.189899 116.04) (end 130.129649 93.10025) (width 0.2) (layer "F.Cu") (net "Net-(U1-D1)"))
 (segment (start 101.4 116.04) (end 107.189899 116.04) (width 0.2) (layer "F.Cu") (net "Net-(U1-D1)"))
 (segment (start 144.25175 114.433) (end 160.5045 98.18025) (width 0.2) (layer "F.Cu") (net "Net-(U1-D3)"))
 (segment (start 144.25175 129.161555) (end 144.25175 114.433) (width 0.2) (layer "F.Cu") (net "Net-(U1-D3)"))
 (segment (start 193.127716 116.21) (end 179.473217 129.864499) (width 0.2) (layer "F.Cu") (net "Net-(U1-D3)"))
 (segment (start 144.954693 129.864499) (end 144.25175 129.161555) (width 0.2) (layer "F.Cu") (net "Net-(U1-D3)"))
 (segment (start 200.27 116.21) (end 193.127716 116.21) (width 0.2) (layer "F.Cu") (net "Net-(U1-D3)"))
 (segment (start 179.473217 129.864499) (end 144.954693 129.864499) (width 0.2) (layer "F.Cu") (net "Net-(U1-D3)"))
 (segment (start 155.10525 127.3645) (end 176.6695 105.80025) (width 0.2) (layer "F.Cu") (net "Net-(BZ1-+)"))
 (segment (start 146.75175 127.3645) (end 155.10525 127.3645) (width 0.2) (layer "F.Cu") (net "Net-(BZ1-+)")))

